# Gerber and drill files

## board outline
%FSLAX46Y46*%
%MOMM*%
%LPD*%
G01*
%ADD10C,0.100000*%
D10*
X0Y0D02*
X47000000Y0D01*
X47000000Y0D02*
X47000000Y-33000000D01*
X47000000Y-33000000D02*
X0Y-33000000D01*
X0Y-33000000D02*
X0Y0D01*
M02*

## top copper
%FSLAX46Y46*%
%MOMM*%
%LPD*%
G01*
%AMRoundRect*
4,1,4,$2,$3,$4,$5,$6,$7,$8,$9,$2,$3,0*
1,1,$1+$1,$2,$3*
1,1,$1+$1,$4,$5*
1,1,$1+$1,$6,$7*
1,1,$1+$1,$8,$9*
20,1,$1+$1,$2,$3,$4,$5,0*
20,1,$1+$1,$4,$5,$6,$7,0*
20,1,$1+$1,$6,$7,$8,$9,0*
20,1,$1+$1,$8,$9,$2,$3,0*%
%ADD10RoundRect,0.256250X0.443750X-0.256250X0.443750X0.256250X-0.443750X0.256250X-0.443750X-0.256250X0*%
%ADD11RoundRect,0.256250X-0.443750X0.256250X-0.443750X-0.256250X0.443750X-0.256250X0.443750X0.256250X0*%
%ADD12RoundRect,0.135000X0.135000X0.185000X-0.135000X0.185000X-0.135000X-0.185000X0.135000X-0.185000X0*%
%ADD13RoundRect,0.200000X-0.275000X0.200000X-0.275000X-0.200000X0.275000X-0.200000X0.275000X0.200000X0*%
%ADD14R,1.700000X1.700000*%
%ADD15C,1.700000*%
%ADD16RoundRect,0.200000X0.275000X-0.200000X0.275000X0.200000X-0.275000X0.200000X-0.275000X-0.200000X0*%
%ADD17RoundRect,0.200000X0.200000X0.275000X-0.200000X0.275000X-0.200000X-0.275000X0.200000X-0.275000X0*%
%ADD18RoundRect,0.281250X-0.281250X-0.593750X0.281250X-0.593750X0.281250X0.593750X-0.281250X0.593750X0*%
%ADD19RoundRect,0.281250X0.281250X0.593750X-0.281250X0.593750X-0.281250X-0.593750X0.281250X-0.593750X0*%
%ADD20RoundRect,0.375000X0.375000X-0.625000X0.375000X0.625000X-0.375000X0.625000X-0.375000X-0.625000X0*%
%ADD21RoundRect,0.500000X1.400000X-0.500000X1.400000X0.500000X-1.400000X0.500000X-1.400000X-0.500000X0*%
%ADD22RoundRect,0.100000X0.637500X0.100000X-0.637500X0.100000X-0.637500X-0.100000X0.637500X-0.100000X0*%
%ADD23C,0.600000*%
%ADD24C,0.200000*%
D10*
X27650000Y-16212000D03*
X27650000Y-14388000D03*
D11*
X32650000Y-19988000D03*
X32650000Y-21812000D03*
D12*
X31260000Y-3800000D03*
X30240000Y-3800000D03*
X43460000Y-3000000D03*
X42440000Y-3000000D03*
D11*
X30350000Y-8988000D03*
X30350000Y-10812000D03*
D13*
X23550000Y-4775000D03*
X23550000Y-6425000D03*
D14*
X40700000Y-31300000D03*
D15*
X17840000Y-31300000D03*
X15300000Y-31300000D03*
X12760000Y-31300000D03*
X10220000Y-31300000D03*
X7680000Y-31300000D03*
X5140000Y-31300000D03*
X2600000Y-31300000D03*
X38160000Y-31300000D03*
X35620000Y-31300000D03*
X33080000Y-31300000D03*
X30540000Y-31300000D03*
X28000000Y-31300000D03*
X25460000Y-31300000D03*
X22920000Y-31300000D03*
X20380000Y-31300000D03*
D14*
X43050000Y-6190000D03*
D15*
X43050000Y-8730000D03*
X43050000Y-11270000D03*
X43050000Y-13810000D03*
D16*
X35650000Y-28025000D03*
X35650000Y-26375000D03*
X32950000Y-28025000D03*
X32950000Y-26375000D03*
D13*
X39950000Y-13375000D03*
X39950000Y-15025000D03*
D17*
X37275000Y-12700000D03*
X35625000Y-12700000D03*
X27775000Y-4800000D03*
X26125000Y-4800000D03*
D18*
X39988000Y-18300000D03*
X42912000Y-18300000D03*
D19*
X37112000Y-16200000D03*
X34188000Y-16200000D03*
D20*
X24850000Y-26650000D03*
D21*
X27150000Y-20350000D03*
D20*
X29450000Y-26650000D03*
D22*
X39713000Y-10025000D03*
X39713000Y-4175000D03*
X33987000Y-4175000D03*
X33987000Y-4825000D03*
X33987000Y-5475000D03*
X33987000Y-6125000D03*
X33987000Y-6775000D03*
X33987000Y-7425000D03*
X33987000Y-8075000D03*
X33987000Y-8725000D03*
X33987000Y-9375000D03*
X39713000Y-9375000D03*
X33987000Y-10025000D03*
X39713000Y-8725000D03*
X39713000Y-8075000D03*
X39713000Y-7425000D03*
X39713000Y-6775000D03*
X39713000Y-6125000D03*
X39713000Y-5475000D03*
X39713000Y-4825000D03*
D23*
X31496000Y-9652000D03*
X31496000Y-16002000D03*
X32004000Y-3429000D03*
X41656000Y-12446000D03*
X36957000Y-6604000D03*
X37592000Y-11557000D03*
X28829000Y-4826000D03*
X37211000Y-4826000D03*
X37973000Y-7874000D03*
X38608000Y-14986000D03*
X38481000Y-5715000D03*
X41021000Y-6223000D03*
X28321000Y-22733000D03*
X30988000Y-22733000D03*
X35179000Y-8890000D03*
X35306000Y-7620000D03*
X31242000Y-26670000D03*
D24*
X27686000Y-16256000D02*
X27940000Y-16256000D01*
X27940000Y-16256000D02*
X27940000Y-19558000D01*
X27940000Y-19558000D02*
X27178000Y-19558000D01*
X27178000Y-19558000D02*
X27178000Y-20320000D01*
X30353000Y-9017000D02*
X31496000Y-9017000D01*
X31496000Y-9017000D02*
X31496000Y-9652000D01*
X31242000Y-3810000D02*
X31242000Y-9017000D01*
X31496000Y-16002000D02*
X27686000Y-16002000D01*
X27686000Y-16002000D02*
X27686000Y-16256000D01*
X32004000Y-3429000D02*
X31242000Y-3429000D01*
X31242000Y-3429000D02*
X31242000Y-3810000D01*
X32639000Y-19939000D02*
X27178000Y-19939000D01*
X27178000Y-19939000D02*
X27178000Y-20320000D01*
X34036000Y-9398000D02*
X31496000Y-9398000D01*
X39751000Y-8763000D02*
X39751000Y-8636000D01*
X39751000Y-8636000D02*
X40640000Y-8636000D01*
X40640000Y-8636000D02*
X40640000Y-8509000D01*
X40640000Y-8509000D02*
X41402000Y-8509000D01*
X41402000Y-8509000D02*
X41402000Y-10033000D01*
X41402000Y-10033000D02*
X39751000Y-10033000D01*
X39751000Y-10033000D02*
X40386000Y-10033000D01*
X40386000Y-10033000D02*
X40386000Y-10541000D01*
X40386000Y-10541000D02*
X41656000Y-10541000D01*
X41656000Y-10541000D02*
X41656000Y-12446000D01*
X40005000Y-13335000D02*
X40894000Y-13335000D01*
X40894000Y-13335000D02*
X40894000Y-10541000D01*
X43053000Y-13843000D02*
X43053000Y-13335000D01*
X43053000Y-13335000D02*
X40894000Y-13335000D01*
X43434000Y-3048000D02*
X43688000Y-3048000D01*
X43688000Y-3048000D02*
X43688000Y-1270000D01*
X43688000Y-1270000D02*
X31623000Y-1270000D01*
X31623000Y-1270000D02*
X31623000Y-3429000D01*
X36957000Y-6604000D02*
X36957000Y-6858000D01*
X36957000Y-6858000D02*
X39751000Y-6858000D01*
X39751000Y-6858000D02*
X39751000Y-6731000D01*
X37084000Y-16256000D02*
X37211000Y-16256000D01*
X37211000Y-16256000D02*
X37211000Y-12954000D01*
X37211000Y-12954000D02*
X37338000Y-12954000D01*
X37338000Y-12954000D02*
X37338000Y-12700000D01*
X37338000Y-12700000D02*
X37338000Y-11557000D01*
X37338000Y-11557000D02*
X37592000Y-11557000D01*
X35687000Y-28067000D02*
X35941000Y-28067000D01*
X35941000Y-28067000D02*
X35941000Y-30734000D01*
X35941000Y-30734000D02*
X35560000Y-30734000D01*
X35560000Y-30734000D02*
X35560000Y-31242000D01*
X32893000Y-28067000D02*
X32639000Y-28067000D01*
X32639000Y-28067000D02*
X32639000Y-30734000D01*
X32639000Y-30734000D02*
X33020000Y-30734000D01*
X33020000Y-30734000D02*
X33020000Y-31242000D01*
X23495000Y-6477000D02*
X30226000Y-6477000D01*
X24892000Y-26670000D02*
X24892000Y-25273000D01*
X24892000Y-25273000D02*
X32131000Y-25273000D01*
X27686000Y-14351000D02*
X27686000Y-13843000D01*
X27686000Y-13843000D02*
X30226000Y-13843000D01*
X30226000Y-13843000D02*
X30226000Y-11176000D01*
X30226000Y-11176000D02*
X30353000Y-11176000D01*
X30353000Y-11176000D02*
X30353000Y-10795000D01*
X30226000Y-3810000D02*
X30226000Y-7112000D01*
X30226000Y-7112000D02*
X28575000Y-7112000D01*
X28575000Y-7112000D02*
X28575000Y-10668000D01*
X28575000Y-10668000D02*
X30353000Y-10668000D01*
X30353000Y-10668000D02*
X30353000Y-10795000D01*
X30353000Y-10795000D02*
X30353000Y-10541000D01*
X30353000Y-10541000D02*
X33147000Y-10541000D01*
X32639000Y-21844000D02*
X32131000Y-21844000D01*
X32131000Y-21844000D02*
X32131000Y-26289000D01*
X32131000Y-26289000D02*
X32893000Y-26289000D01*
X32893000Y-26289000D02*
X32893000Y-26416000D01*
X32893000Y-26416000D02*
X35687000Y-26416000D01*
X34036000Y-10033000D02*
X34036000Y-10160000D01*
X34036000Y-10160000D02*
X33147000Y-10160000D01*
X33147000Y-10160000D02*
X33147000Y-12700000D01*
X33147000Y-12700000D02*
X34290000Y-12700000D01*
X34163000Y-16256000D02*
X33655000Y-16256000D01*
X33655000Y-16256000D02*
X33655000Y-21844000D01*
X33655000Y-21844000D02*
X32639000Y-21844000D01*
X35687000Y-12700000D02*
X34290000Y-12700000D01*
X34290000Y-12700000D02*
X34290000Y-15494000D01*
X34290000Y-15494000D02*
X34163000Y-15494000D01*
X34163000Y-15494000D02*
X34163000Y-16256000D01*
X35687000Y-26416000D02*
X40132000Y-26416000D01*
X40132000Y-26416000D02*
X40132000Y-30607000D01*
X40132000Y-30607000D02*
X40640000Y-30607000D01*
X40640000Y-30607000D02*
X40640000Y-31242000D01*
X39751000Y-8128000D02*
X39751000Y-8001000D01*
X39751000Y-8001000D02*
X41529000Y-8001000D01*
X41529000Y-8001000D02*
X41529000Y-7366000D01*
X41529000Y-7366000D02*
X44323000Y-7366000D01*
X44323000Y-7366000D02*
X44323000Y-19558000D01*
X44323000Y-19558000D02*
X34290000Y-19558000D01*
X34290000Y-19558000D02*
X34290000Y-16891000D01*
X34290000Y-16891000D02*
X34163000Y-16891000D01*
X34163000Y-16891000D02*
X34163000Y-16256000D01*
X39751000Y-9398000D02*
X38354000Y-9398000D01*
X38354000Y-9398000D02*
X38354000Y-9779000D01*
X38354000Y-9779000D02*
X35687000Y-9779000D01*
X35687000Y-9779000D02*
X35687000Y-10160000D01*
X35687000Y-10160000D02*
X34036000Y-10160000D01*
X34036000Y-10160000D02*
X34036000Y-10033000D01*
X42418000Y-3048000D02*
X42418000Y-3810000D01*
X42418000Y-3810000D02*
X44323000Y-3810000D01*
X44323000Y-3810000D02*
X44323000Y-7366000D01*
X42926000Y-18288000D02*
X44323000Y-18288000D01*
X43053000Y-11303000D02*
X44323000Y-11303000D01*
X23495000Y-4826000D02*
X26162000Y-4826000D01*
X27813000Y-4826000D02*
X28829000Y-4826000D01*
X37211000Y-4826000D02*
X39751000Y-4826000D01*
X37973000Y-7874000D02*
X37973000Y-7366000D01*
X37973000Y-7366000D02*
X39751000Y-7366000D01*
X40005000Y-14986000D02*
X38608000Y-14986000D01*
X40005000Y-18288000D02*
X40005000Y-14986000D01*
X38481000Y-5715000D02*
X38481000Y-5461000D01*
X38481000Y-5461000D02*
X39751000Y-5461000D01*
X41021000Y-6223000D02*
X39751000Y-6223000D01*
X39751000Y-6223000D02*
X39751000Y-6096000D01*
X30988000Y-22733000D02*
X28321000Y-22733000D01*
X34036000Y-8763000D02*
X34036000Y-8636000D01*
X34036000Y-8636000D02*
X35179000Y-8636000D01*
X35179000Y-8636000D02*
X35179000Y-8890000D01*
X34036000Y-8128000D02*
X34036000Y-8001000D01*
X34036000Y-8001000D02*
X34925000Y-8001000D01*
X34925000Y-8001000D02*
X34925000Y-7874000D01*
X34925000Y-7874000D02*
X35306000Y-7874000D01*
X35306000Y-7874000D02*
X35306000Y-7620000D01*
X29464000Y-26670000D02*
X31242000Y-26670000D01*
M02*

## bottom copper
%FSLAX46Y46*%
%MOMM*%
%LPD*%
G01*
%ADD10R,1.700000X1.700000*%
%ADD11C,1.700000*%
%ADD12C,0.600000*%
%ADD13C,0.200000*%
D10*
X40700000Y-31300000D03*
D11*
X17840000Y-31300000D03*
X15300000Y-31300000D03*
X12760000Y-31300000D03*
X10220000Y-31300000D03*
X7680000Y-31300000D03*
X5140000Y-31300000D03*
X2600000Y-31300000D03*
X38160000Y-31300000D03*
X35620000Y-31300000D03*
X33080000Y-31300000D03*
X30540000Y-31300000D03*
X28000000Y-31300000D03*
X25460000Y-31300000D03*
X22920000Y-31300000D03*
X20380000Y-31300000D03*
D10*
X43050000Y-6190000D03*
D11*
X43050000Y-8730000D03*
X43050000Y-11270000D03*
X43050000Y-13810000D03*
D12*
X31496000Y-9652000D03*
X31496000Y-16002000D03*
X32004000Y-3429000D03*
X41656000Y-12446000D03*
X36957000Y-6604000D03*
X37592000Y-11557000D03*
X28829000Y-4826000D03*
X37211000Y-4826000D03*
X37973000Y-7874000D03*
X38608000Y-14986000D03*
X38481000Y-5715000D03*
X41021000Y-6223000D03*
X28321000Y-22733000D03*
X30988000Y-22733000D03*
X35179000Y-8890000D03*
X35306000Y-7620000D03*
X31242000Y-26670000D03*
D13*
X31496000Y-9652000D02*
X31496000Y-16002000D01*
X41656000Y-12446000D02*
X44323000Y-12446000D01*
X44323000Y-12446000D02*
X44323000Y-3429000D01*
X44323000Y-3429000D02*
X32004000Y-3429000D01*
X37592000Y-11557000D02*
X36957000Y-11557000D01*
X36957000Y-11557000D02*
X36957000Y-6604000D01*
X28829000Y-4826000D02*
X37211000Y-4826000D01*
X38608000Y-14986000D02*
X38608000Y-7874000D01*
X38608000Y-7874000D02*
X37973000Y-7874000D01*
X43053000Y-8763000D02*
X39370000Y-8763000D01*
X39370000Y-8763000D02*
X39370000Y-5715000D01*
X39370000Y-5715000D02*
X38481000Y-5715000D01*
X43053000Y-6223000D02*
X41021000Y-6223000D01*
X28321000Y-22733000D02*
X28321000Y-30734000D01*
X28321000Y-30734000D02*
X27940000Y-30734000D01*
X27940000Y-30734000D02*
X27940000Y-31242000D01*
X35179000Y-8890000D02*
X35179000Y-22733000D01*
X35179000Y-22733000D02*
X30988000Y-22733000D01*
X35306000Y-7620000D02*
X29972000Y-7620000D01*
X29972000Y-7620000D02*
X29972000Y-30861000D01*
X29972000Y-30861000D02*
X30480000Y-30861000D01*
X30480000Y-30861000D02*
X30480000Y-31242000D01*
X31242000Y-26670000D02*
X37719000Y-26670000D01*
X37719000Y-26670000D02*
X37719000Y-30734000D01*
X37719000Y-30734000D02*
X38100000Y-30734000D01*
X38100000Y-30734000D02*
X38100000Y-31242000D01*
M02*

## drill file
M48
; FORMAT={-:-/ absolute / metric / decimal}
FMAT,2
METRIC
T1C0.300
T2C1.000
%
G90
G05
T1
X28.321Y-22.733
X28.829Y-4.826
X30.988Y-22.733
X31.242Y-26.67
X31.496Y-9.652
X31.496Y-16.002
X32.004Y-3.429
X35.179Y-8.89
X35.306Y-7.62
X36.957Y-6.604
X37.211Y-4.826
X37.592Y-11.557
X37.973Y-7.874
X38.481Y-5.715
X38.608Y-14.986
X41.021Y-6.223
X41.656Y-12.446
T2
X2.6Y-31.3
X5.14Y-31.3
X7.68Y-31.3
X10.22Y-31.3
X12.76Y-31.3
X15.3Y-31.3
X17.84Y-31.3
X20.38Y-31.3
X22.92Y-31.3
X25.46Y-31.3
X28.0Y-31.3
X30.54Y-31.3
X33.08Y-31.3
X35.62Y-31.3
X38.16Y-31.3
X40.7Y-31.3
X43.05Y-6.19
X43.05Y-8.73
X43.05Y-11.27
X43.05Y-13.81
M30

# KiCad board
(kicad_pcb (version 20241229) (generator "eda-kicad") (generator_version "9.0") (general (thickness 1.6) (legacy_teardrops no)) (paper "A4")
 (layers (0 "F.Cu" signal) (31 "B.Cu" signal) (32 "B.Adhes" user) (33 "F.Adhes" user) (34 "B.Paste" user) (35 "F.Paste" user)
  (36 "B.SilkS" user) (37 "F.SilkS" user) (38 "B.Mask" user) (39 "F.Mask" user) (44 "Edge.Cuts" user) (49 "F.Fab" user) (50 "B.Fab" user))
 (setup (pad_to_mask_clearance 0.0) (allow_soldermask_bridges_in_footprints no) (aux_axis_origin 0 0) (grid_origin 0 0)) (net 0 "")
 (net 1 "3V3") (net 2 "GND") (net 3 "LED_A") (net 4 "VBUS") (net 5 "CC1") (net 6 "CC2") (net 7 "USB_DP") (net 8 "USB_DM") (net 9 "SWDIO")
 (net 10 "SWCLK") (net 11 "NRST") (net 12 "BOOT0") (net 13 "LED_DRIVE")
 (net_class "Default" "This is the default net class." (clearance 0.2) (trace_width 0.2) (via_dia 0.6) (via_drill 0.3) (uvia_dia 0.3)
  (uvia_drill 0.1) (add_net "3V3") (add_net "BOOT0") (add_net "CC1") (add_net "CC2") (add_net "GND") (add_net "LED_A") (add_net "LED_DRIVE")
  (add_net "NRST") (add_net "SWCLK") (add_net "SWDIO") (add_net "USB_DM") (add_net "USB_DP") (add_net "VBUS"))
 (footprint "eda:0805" (layer "F.Cu") (at 27.65 15.3 -270)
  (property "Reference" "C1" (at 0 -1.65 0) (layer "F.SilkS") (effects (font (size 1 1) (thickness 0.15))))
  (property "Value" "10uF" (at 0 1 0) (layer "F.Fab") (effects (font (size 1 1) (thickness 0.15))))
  (pad "1" smd roundrect (at -0.912 0 -270) (size 1.025 1.4) (roundrect_rratio 0.25) (layers "F.Cu" "F.Paste" "F.Mask") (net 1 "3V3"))
  (pad "2" smd roundrect (at 0.912 0 -270) (size 1.025 1.4) (roundrect_rratio 0.25) (layers "F.Cu" "F.Paste" "F.Mask") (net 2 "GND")))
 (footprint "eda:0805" (layer "F.Cu") (at 32.65 20.9 -90)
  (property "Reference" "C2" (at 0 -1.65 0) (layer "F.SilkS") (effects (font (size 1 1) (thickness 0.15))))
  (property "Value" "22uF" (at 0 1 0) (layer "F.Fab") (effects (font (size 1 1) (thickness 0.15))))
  (pad "1" smd roundrect (at -0.912 0 -90) (size 1.025 1.4) (roundrect_rratio 0.25) (layers "F.Cu" "F.Paste" "F.Mask") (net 1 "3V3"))
  (pad "2" smd roundrect (at 0.912 0 -90) (size 1.025 1.4) (roundrect_rratio 0.25) (layers "F.Cu" "F.Paste" "F.Mask") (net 2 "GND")))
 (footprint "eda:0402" (layer "F.Cu") (at 30.75 3.8 -180)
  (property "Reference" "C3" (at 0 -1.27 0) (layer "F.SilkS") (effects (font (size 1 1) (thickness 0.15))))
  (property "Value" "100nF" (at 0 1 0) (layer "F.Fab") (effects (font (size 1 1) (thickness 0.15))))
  (pad "1" smd roundrect (at -0.51 0 -180) (size 0.54 0.64) (roundrect_rratio 0.25) (layers "F.Cu" "F.Paste" "F.Mask") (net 1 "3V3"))
  (pad "2" smd roundrect (at 0.51 0 -180) (size 0.54 0.64) (roundrect_rratio 0.25) (layers "F.Cu" "F.Paste" "F.Mask") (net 2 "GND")))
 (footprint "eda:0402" (layer "F.Cu") (at 42.95 3 -180)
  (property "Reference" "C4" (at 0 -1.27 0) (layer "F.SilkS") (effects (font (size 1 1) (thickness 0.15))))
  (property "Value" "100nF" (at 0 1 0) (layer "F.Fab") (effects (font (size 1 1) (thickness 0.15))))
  (pad "1" smd roundrect (at -0.51 0 -180) (size 0.54 0.64) (roundrect_rratio 0.25) (layers "F.Cu" "F.Paste" "F.Mask") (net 1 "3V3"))
  (pad "2" smd roundrect (at 0.51 0 -180) (size 0.54 0.64) (roundrect_rratio 0.25) (layers "F.Cu" "F.Paste" "F.Mask") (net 2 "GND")))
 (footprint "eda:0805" (layer "F.Cu") (at 30.35 9.9 -90)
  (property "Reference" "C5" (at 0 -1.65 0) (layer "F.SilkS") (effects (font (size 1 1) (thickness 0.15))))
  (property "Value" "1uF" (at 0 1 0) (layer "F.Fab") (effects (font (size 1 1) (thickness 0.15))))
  (pad "1" smd roundrect (at -0.912 0 -90) (size 1.025 1.4) (roundrect_rratio 0.25) (layers "F.Cu" "F.Paste" "F.Mask") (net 1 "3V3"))
  (pad "2" smd roundrect (at 0.912 0 -90) (size 1.025 1.4) (roundrect_rratio 0.25) (layers "F.Cu" "F.Paste" "F.Mask") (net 2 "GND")))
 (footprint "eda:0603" (layer "F.Cu") (at 23.55 5.6 -90)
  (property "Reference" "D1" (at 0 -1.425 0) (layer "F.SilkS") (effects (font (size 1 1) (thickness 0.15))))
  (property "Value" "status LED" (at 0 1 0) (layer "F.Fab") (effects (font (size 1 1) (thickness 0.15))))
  (pad "1" smd roundrect (at -0.825 0 -90) (size 0.8 0.95) (roundrect_rratio 0.25) (layers "F.Cu" "F.Paste" "F.Mask") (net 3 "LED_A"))
  (pad "2" smd roundrect (at 0.825 0 -90) (size 0.8 0.95) (roundrect_rratio 0.25) (layers "F.Cu" "F.Paste" "F.Mask") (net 2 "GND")))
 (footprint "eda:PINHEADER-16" (layer "F.Cu") (at 21.65 31.3 -180)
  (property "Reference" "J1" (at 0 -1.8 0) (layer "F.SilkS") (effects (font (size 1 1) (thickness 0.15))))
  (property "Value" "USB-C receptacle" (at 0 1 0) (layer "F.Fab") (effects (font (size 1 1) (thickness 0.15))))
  (pad "1" thru_hole rect (at -19.05 0 -180) (size 1.7 1.7) (drill 1) (layers "*.Cu" "*.Mask") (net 2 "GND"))
  (pad "10" thru_hole circle (at 3.81 0 -180) (size 1.7 1.7) (drill 1) (layers "*.Cu" "*.Mask"))
  (pad "11" thru_hole circle (at 6.35 0 -180) (size 1.7 1.7) (drill 1) (layers "*.Cu" "*.Mask"))
  (pad "12" thru_hole circle (at 8.89 0 -180) (size 1.7 1.7) (drill 1) (layers "*.Cu" "*.Mask"))
  (pad "13" thru_hole circle (at 11.43 0 -180) (size 1.7 1.7) (drill 1) (layers "*.Cu" "*.Mask"))
  (pad "14" thru_hole circle (at 13.97 0 -180) (size 1.7 1.7) (drill 1) (layers "*.Cu" "*.Mask"))
  (pad "15" thru_hole circle (at 16.51 0 -180) (size 1.7 1.7) (drill 1) (layers "*.Cu" "*.Mask"))
  (pad "16" thru_hole circle (at 19.05 0 -180) (size 1.7 1.7) (drill 1) (layers "*.Cu" "*.Mask"))
  (pad "2" thru_hole circle (at -16.51 0 -180) (size 1.7 1.7) (drill 1) (layers "*.Cu" "*.Mask") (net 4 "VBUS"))
  (pad "3" thru_hole circle (at -13.97 0 -180) (size 1.7 1.7) (drill 1) (layers "*.Cu" "*.Mask") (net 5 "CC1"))
  (pad "4" thru_hole circle (at -11.43 0 -180) (size 1.7 1.7) (drill 1) (layers "*.Cu" "*.Mask") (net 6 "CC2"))
  (pad "5" thru_hole circle (at -8.89 0 -180) (size 1.7 1.7) (drill 1) (layers "*.Cu" "*.Mask") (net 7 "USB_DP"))
  (pad "6" thru_hole circle (at -6.35 0 -180) (size 1.7 1.7) (drill 1) (layers "*.Cu" "*.Mask") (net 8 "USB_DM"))
  (pad "7" thru_hole circle (at -3.81 0 -180) (size 1.7 1.7) (drill 1) (layers "*.Cu" "*.Mask"))
  (pad "8" thru_hole circle (at -1.27 0 -180) (size 1.7 1.7) (drill 1) (layers "*.Cu" "*.Mask"))
  (pad "9" thru_hole circle (at 1.27 0 -180) (size 1.7 1.7) (drill 1) (layers "*.Cu" "*.Mask")))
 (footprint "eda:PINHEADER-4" (layer "F.Cu") (at 43.05 10 -90)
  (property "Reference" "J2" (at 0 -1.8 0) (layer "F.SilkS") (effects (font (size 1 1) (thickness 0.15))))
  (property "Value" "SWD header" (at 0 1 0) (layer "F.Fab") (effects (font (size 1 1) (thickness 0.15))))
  (pad "1" thru_hole rect (at -3.81 0 -90) (size 1.7 1.7) (drill 1) (layers "*.Cu" "*.Mask") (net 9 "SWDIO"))
  (pad "2" thru_hole circle (at -1.27 0 -90) (size 1.7 1.7) (drill 1) (layers "*.Cu" "*.Mask") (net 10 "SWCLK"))
  (pad "3" thru_hole circle (at 1.27 0 -90) (size 1.7 1.7) (drill 1) (layers "*.Cu" "*.Mask") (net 2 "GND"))
  (pad "4" thru_hole circle (at 3.81 0 -90) (size 1.7 1.7) (drill 1) (layers "*.Cu" "*.Mask") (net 1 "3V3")))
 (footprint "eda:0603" (layer "F.Cu") (at 35.65 27.2 -270)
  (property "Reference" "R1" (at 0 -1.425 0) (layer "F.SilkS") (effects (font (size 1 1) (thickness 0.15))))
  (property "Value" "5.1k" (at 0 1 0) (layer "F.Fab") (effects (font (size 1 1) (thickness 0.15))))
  (pad "1" smd roundrect (at -0.825 0 -270) (size 0.8 0.95) (roundrect_rratio 0.25) (layers "F.Cu" "F.Paste" "F.Mask") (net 5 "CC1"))
  (pad "2" smd roundrect (at 0.825 0 -270) (size 0.8 0.95) (roundrect_rratio 0.25) (layers "F.Cu" "F.Paste" "F.Mask") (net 2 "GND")))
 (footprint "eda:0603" (layer "F.Cu") (at 32.95 27.2 -270)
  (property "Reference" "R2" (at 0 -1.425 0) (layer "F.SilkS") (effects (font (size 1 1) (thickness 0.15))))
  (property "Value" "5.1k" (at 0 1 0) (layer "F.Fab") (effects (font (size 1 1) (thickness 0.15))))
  (pad "1" smd roundrect (at -0.825 0 -270) (size 0.8 0.95) (roundrect_rratio 0.25) (layers "F.Cu" "F.Paste" "F.Mask") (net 6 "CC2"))
  (pad "2" smd roundrect (at 0.825 0 -270) (size 0.8 0.95) (roundrect_rratio 0.25) (layers "F.Cu" "F.Paste" "F.Mask") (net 2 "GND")))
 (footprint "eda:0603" (layer "F.Cu") (at 39.95 14.2 -90)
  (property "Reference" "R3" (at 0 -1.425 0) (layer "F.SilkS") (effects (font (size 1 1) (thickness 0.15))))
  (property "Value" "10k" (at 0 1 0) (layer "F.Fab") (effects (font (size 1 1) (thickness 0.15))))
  (pad "1" smd roundrect (at -0.825 0 -90) (size 0.8 0.95) (roundrect_rratio 0.25) (layers "F.Cu" "F.Paste" "F.Mask") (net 1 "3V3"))
  (pad "2" smd roundrect (at 0.825 0 -90) (size 0.8 0.95) (roundrect_rratio 0.25) (layers "F.Cu" "F.Paste" "F.Mask") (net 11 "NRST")))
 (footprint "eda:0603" (layer "F.Cu") (at 36.45 12.7 -180)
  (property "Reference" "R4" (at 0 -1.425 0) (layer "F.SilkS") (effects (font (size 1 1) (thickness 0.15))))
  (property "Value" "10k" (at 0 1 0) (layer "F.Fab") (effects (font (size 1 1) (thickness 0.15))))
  (pad "1" smd roundrect (at -0.825 0 -180) (size 0.8 0.95) (roundrect_rratio 0.25) (layers "F.Cu" "F.Paste" "F.Mask") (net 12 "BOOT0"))
  (pad "2" smd roundrect (at 0.825 0 -180) (size 0.8 0.95) (roundrect_rratio 0.25) (layers "F.Cu" "F.Paste" "F.Mask") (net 2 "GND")))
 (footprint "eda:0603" (layer "F.Cu") (at 26.95 4.8 -180)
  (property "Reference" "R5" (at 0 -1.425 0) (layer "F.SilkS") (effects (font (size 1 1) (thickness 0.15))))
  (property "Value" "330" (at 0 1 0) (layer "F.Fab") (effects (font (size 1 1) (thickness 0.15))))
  (pad "1" smd roundrect (at -0.825 0 -180) (size 0.8 0.95) (roundrect_rratio 0.25) (layers "F.Cu" "F.Paste" "F.Mask") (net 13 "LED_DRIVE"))
  (pad "2" smd roundrect (at 0.825 0 -180) (size 0.8 0.95) (roundrect_rratio 0.25) (layers "F.Cu" "F.Paste" "F.Mask") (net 3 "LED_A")))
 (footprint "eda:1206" (layer "F.Cu") (at 41.45 18.3 0)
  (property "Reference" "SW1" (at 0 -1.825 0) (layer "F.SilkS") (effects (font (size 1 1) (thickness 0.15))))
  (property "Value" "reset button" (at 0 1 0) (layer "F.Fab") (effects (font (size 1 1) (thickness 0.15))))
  (pad "1" smd roundrect (at -1.462 0 0) (size 1.125 1.75) (roundrect_rratio 0.25) (layers "F.Cu" "F.Paste" "F.Mask") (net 11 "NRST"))
  (pad "2" smd roundrect (at 1.462 0 0) (size 1.125 1.75) (roundrect_rratio 0.25) (layers "F.Cu" "F.Paste" "F.Mask") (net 2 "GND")))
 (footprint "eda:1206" (layer "F.Cu") (at 35.65 16.2 -180)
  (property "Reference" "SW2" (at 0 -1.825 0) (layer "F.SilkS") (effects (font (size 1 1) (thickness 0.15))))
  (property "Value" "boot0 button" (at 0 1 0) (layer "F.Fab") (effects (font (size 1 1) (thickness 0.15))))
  (pad "1" smd roundrect (at -1.462 0 -180) (size 1.125 1.75) (roundrect_rratio 0.25) (layers "F.Cu" "F.Paste" "F.Mask") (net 12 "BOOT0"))
  (pad "2" smd roundrect (at 1.462 0 -180) (size 1.125 1.75) (roundrect_rratio 0.25) (layers "F.Cu" "F.Paste" "F.Mask") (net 2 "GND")))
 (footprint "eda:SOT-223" (layer "F.Cu") (at 27.15 23.5 -270)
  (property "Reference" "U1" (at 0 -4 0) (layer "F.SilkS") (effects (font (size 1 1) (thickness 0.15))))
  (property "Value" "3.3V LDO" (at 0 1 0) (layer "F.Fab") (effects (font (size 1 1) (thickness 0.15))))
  (pad "1" smd roundrect (at -3.15 -2.3 -270) (size 2 1.5) (roundrect_rratio 0.25) (layers "F.Cu" "F.Paste" "F.Mask") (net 2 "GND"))
  (pad "2" smd roundrect (at 3.15 0 -270) (size 2 3.8) (roundrect_rratio 0.25) (layers "F.Cu" "F.Paste" "F.Mask") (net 1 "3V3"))
  (pad "3" smd roundrect (at -3.15 2.3 -270) (size 2 1.5) (roundrect_rratio 0.25) (layers "F.Cu" "F.Paste" "F.Mask") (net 4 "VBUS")))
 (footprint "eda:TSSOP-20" (layer "F.Cu") (at 36.85 7.1 -180)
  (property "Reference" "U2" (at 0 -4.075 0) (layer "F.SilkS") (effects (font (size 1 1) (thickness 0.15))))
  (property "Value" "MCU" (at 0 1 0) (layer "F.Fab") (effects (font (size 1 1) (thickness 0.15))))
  (pad "1" smd roundrect (at -2.863 -2.925 -180) (size 1.475 0.4) (roundrect_rratio 0.25) (layers "F.Cu" "F.Paste" "F.Mask") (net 1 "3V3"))
  (pad "10" smd roundrect (at -2.863 2.925 -180) (size 1.475 0.4) (roundrect_rratio 0.25) (layers "F.Cu" "F.Paste" "F.Mask"))
  (pad "11" smd roundrect (at 2.863 2.925 -180) (size 1.475 0.4) (roundrect_rratio 0.25) (layers "F.Cu" "F.Paste" "F.Mask"))
  (pad "12" smd roundrect (at 2.863 2.275 -180) (size 1.475 0.4) (roundrect_rratio 0.25) (layers "F.Cu" "F.Paste" "F.Mask"))
  (pad "13" smd roundrect (at 2.863 1.625 -180) (size 1.475 0.4) (roundrect_rratio 0.25) (layers "F.Cu" "F.Paste" "F.Mask"))
  (pad "14" smd roundrect (at 2.863 0.975 -180) (size 1.475 0.4) (roundrect_rratio 0.25) (layers "F.Cu" "F.Paste" "F.Mask"))
  (pad "15" smd roundrect (at 2.863 0.325 -180) (size 1.475 0.4) (roundrect_rratio 0.25) (layers "F.Cu" "F.Paste" "F.Mask"))
  (pad "16" smd roundrect (at 2.863 -0.325 -180) (size 1.475 0.4) (roundrect_rratio 0.25) (layers "F.Cu" "F.Paste" "F.Mask"))
  (pad "17" smd roundrect (at 2.863 -0.975 -180) (size 1.475 0.4) (roundrect_rratio 0.25) (layers "F.Cu" "F.Paste" "F.Mask")
   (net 7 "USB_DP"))
  (pad "18" smd roundrect (at 2.863 -1.625 -180) (size 1.475 0.4) (roundrect_rratio 0.25) (layers "F.Cu" "F.Paste" "F.Mask")
   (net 8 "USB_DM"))
  (pad "19" smd roundrect (at 2.863 -2.275 -180) (size 1.475 0.4) (roundrect_rratio 0.25) (layers "F.Cu" "F.Paste" "F.Mask") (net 1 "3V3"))
  (pad "2" smd roundrect (at -2.863 -2.275 -180) (size 1.475 0.4) (roundrect_rratio 0.25) (layers "F.Cu" "F.Paste" "F.Mask") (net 2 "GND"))
  (pad "20" smd roundrect (at 2.863 -2.925 -180) (size 1.475 0.4) (roundrect_rratio 0.25) (layers "F.Cu" "F.Paste" "F.Mask") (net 2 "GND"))
  (pad "3" smd roundrect (at -2.863 -1.625 -180) (size 1.475 0.4) (roundrect_rratio 0.25) (layers "F.Cu" "F.Paste" "F.Mask") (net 1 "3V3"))
  (pad "4" smd roundrect (at -2.863 -0.975 -180) (size 1.475 0.4) (roundrect_rratio 0.25) (layers "F.Cu" "F.Paste" "F.Mask") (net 2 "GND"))
  (pad "5" smd roundrect (at -2.863 -0.325 -180) (size 1.475 0.4) (roundrect_rratio 0.25) (layers "F.Cu" "F.Paste" "F.Mask") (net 11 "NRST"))
  (pad "6" smd roundrect (at -2.863 0.325 -180) (size 1.475 0.4) (roundrect_rratio 0.25) (layers "F.Cu" "F.Paste" "F.Mask") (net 12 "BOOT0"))
  (pad "7" smd roundrect (at -2.863 0.975 -180) (size 1.475 0.4) (roundrect_rratio 0.25) (layers "F.Cu" "F.Paste" "F.Mask") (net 9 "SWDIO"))
  (pad "8" smd roundrect (at -2.863 1.625 -180) (size 1.475 0.4) (roundrect_rratio 0.25) (layers "F.Cu" "F.Paste" "F.Mask") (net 10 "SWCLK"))
  (pad "9" smd roundrect (at -2.863 2.275 -180) (size 1.475 0.4) (roundrect_rratio 0.25) (layers "F.Cu" "F.Paste" "F.Mask")
   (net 13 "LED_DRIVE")))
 (segment (start 31.496 9.652) (end 31.496 16.002) (width 0.2) (layer "B.Cu") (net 1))
 (segment (start 41.656 12.446) (end 44.323 12.446) (width 0.2) (layer "B.Cu") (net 1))
 (segment (start 44.323 12.446) (end 44.323 3.429) (width 0.2) (layer "B.Cu") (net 1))
 (segment (start 44.323 3.429) (end 32.004 3.429) (width 0.2) (layer "B.Cu") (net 1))
 (segment (start 27.686 16.256) (end 27.94 16.256) (width 0.2) (layer "F.Cu") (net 1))
 (segment (start 27.94 16.256) (end 27.94 19.558) (width 0.2) (layer "F.Cu") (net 1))
 (segment (start 27.94 19.558) (end 27.178 19.558) (width 0.2) (layer "F.Cu") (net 1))
 (segment (start 27.178 19.558) (end 27.178 20.32) (width 0.2) (layer "F.Cu") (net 1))
 (segment (start 30.353 9.017) (end 31.496 9.017) (width 0.2) (layer "F.Cu") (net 1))
 (segment (start 31.496 9.017) (end 31.496 9.652) (width 0.2) (layer "F.Cu") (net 1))
 (segment (start 31.242 3.81) (end 31.242 9.017) (width 0.2) (layer "F.Cu") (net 1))
 (segment (start 31.496 16.002) (end 27.686 16.002) (width 0.2) (layer "F.Cu") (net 1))
 (segment (start 27.686 16.002) (end 27.686 16.256) (width 0.2) (layer "F.Cu") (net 1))
 (segment (start 32.004 3.429) (end 31.242 3.429) (width 0.2) (layer "F.Cu") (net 1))
 (segment (start 31.242 3.429) (end 31.242 3.81) (width 0.2) (layer "F.Cu") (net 1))
 (segment (start 32.639 19.939) (end 27.178 19.939) (width 0.2) (layer "F.Cu") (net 1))
 (segment (start 27.178 19.939) (end 27.178 20.32) (width 0.2) (layer "F.Cu") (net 1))
 (segment (start 34.036 9.398) (end 31.496 9.398) (width 0.2) (layer "F.Cu") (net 1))
 (segment (start 39.751 8.763) (end 39.751 8.636) (width 0.2) (layer "F.Cu") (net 1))
 (segment (start 39.751 8.636) (end 40.64 8.636) (width 0.2) (layer "F.Cu") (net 1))
 (segment (start 40.64 8.636) (end 40.64 8.509) (width 0.2) (layer "F.Cu") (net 1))
 (segment (start 40.64 8.509) (end 41.402 8.509) (width 0.2) (layer "F.Cu") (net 1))
 (segment (start 41.402 8.509) (end 41.402 10.033) (width 0.2) (layer "F.Cu") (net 1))
 (segment (start 41.402 10.033) (end 39.751 10.033) (width 0.2) (layer "F.Cu") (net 1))
 (segment (start 39.751 10.033) (end 40.386 10.033) (width 0.2) (layer "F.Cu") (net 1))
 (segment (start 40.386 10.033) (end 40.386 10.541) (width 0.2) (layer "F.Cu") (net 1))
 (segment (start 40.386 10.541) (end 41.656 10.541) (width 0.2) (layer "F.Cu") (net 1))
 (segment (start 41.656 10.541) (end 41.656 12.446) (width 0.2) (layer "F.Cu") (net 1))
 (segment (start 40.005 13.335) (end 40.894 13.335) (width 0.2) (layer "F.Cu") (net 1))
 (segment (start 40.894 13.335) (end 40.894 10.541) (width 0.2) (layer "F.Cu") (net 1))
 (segment (start 43.053 13.843) (end 43.053 13.335) (width 0.2) (layer "F.Cu") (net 1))
 (segment (start 43.053 13.335) (end 40.894 13.335) (width 0.2) (layer "F.Cu") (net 1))
 (segment (start 43.434 3.048) (end 43.688 3.048) (width 0.2) (layer "F.Cu") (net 1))
 (segment (start 43.688 3.048) (end 43.688 1.27) (width 0.2) (layer "F.Cu") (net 1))
 (segment (start 43.688 1.27) (end 31.623 1.27) (width 0.2) (layer "F.Cu") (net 1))
 (segment (start 31.623 1.27) (end 31.623 3.429) (width 0.2) (layer "F.Cu") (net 1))
 (segment (start 37.592 11.557) (end 36.957 11.557) (width 0.2) (layer "B.Cu") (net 12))
 (segment (start 36.957 11.557) (end 36.957 6.604) (width 0.2) (layer "B.Cu") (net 12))
 (segment (start 36.957 6.604) (end 36.957 6.858) (width 0.2) (layer "F.Cu") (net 12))
 (segment (start 36.957 6.858) (end 39.751 6.858) (width 0.2) (layer "F.Cu") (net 12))
 (segment (start 39.751 6.858) (end 39.751 6.731) (width 0.2) (layer "F.Cu") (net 12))
 (segment (start 37.084 16.256) (end 37.211 16.256) (width 0.2) (layer "F.Cu") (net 12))
 (segment (start 37.211 16.256) (end 37.211 12.954) (width 0.2) (layer "F.Cu") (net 12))
 (segment (start 37.211 12.954) (end 37.338 12.954) (width 0.2) (layer "F.Cu") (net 12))
 (segment (start 37.338 12.954) (end 37.338 12.7) (width 0.2) (layer "F.Cu") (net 12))
 (segment (start 37.338 12.7) (end 37.338 11.557) (width 0.2) (layer "F.Cu") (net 12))
 (segment (start 37.338 11.557) (end 37.592 11.557) (width 0.2) (layer "F.Cu") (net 12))
 (segment (start 35.687 28.067) (end 35.941 28.067) (width 0.2) (layer "F.Cu") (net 5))
 (segment (start 35.941 28.067) (end 35.941 30.734) (width 0.2) (layer "F.Cu") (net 5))
 (segment (start 35.941 30.734) (end 35.56 30.734) (width 0.2) (layer "F.Cu") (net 5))
 (segment (start 35.56 30.734) (end 35.56 31.242) (width 0.2) (layer "F.Cu") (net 5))
 (segment (start 32.893 28.067) (end 32.639 28.067) (width 0.2) (layer "F.Cu") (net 6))
 (segment (start 32.639 28.067) (end 32.639 30.734) (width 0.2) (layer "F.Cu") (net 6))
 (segment (start 32.639 30.734) (end 33.02 30.734) (width 0.2) (layer "F.Cu") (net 6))
 (segment (start 33.02 30.734) (end 33.02 31.242) (width 0.2) (layer "F.Cu") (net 6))
 (segment (start 23.495 6.477) (end 30.226 6.477) (width 0.2) (layer "F.Cu") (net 2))
 (segment (start 24.892 26.67) (end 24.892 25.273) (width 0.2) (layer "F.Cu") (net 2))
 (segment (start 24.892 25.273) (end 32.131 25.273) (width 0.2) (layer "F.Cu") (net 2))
 (segment (start 27.686 14.351) (end 27.686 13.843) (width 0.2) (layer "F.Cu") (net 2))
 (segment (start 27.686 13.843) (end 30.226 13.843) (width 0.2) (layer "F.Cu") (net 2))
 (segment (start 30.226 13.843) (end 30.226 11.176) (width 0.2) (layer "F.Cu") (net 2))
 (segment (start 30.226 11.176) (end 30.353 11.176) (width 0.2) (layer "F.Cu") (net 2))
 (segment (start 30.353 11.176) (end 30.353 10.795) (width 0.2) (layer "F.Cu") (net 2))
 (segment (start 30.226 3.81) (end 30.226 7.112) (width 0.2) (layer "F.Cu") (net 2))
 (segment (start 30.226 7.112) (end 28.575 7.112) (width 0.2) (layer "F.Cu") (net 2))
 (segment (start 28.575 7.112) (end 28.575 10.668) (width 0.2) (layer "F.Cu") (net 2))
 (segment (start 28.575 10.668) (end 30.353 10.668) (width 0.2) (layer "F.Cu") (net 2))
 (segment (start 30.353 10.668) (end 30.353 10.795) (width 0.2) (layer "F.Cu") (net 2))
 (segment (start 30.353 10.795) (end 30.353 10.541) (width 0.2) (layer "F.Cu") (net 2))
 (segment (start 30.353 10.541) (end 33.147 10.541) (width 0.2) (layer "F.Cu") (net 2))
 (segment (start 32.639 21.844) (end 32.131 21.844) (width 0.2) (layer "F.Cu") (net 2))
 (segment (start 32.131 21.844) (end 32.131 26.289) (width 0.2) (layer "F.Cu") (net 2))
 (segment (start 32.131 26.289) (end 32.893 26.289) (width 0.2) (layer "F.Cu") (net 2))
 (segment (start 32.893 26.289) (end 32.893 26.416) (width 0.2) (layer "F.Cu") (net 2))
 (segment (start 32.893 26.416) (end 35.687 26.416) (width 0.2) (layer "F.Cu") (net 2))
 (segment (start 34.036 10.033) (end 34.036 10.16) (width 0.2) (layer "F.Cu") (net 2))
 (segment (start 34.036 10.16) (end 33.147 10.16) (width 0.2) (layer "F.Cu") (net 2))
 (segment (start 33.147 10.16) (end 33.147 12.7) (width 0.2) (layer "F.Cu") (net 2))
 (segment (start 33.147 12.7) (end 34.29 12.7) (width 0.2) (layer "F.Cu") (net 2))
 (segment (start 34.163 16.256) (end 33.655 16.256) (width 0.2) (layer "F.Cu") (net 2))
 (segment (start 33.655 16.256) (end 33.655 21.844) (width 0.2) (layer "F.Cu") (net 2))
 (segment (start 33.655 21.844) (end 32.639 21.844) (width 0.2) (layer "F.Cu") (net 2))
 (segment (start 35.687 12.7) (end 34.29 12.7) (width 0.2) (layer "F.Cu") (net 2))
 (segment (start 34.29 12.7) (end 34.29 15.494) (width 0.2) (layer "F.Cu") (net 2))
 (segment (start 34.29 15.494) (end 34.163 15.494) (width 0.2) (layer "F.Cu") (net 2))
 (segment (start 34.163 15.494) (end 34.163 16.256) (width 0.2) (layer "F.Cu") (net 2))
 (segment (start 35.687 26.416) (end 40.132 26.416) (width 0.2) (layer "F.Cu") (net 2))
 (segment (start 40.132 26.416) (end 40.132 30.607) (width 0.2) (layer "F.Cu") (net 2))
 (segment (start 40.132 30.607) (end 40.64 30.607) (width 0.2) (layer "F.Cu") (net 2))
 (segment (start 40.64 30.607) (end 40.64 31.242) (width 0.2) (layer "F.Cu") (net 2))
 (segment (start 39.751 8.128) (end 39.751 8.001) (width 0.2) (layer "F.Cu") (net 2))
 (segment (start 39.751 8.001) (end 41.529 8.001) (width 0.2) (layer "F.Cu") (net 2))
 (segment (start 41.529 8.001) (end 41.529 7.366) (width 0.2) (layer "F.Cu") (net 2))
 (segment (start 41.529 7.366) (end 44.323 7.366) (width 0.2) (layer "F.Cu") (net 2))
 (segment (start 44.323 7.366) (end 44.323 19.558) (width 0.2) (layer "F.Cu") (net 2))
 (segment (start 44.323 19.558) (end 34.29 19.558) (width 0.2) (layer "F.Cu") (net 2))
 (segment (start 34.29 19.558) (end 34.29 16.891) (width 0.2) (layer "F.Cu") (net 2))
 (segment (start 34.29 16.891) (end 34.163 16.891) (width 0.2) (layer "F.Cu") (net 2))
 (segment (start 34.163 16.891) (end 34.163 16.256) (width 0.2) (layer "F.Cu") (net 2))
 (segment (start 39.751 9.398) (end 38.354 9.398) (width 0.2) (layer "F.Cu") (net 2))
 (segment (start 38.354 9.398) (end 38.354 9.779) (width 0.2) (layer "F.Cu") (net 2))
 (segment (start 38.354 9.779) (end 35.687 9.779) (width 0.2) (layer "F.Cu") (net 2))
 (segment (start 35.687 9.779) (end 35.687 10.16) (width 0.2) (layer "F.Cu") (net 2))
 (segment (start 35.687 10.16) (end 34.036 10.16) (width 0.2) (layer "F.Cu") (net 2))
 (segment (start 34.036 10.16) (end 34.036 10.033) (width 0.2) (layer "F.Cu") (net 2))
 (segment (start 42.418 3.048) (end 42.418 3.81) (width 0.2) (layer "F.Cu") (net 2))
 (segment (start 42.418 3.81) (end 44.323 3.81) (width 0.2) (layer "F.Cu") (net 2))
 (segment (start 44.323 3.81) (end 44.323 7.366) (width 0.2) (layer "F.Cu") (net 2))
 (segment (start 42.926 18.288) (end 44.323 18.288) (width 0.2) (layer "F.Cu") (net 2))
 (segment (start 43.053 11.303) (end 44.323 11.303) (width 0.2) (layer "F.Cu") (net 2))
 (segment (start 23.495 4.826) (end 26.162 4.826) (width 0.2) (layer "F.Cu") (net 3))
 (segment (start 28.829 4.826) (end 37.211 4.826) (width 0.2) (layer "B.Cu") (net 13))
 (segment (start 27.813 4.826) (end 28.829 4.826) (width 0.2) (layer "F.Cu") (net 13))
 (segment (start 37.211 4.826) (end 39.751 4.826) (width 0.2) (layer "F.Cu") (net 13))
 (segment (start 38.608 14.986) (end 38.608 7.874) (width 0.2) (layer "B.Cu") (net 11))
 (segment (start 38.608 7.874) (end 37.973 7.874) (width 0.2) (layer "B.Cu") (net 11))
 (segment (start 37.973 7.874) (end 37.973 7.366) (width 0.2) (layer "F.Cu") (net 11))
 (segment (start 37.973 7.366) (end 39.751 7.366) (width 0.2) (layer "F.Cu") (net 11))
 (segment (start 40.005 14.986) (end 38.608 14.986) (width 0.2) (layer "F.Cu") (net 11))
 (segment (start 40.005 18.288) (end 40.005 14.986) (width 0.2) (layer "F.Cu") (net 11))
 (segment (start 43.053 8.763) (end 39.37 8.763) (width 0.2) (layer "B.Cu") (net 10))
 (segment (start 39.37 8.763) (end 39.37 5.715) (width 0.2) (layer "B.Cu") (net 10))
 (segment (start 39.37 5.715) (end 38.481 5.715) (width 0.2) (layer "B.Cu") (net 10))
 (segment (start 38.481 5.715) (end 38.481 5.461) (width 0.2) (layer "F.Cu") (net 10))
 (segment (start 38.481 5.461) (end 39.751 5.461) (width 0.2) (layer "F.Cu") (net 10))
 (segment (start 43.053 6.223) (end 41.021 6.223) (width 0.2) (layer "B.Cu") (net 9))
 (segment (start 41.021 6.223) (end 39.751 6.223) (width 0.2) (layer "F.Cu") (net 9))
 (segment (start 39.751 6.223) (end 39.751 6.096) (width 0.2) (layer "F.Cu") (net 9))
 (segment (start 28.321 22.733) (end 28.321 30.734) (width 0.2) (layer "B.Cu") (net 8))
 (segment (start 28.321 30.734) (end 27.94 30.734) (width 0.2) (layer "B.Cu") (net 8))
 (segment (start 27.94 30.734) (end 27.94 31.242) (width 0.2) (layer "B.Cu") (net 8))
 (segment (start 35.179 8.89) (end 35.179 22.733) (width 0.2) (layer "B.Cu") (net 8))
 (segment (start 35.179 22.733) (end 30.988 22.733) (width 0.2) (layer "B.Cu") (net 8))
 (segment (start 30.988 22.733) (end 28.321 22.733) (width 0.2) (layer "F.Cu") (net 8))
 (segment (start 34.036 8.763) (end 34.036 8.636) (width 0.2) (layer "F.Cu") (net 8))
 (segment (start 34.036 8.636) (end 35.179 8.636) (width 0.2) (layer "F.Cu") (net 8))
 (segment (start 35.179 8.636) (end 35.179 8.89) (width 0.2) (layer "F.Cu") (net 8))
 (segment (start 35.306 7.62) (end 29.972 7.62) (width 0.2) (layer "B.Cu") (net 7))
 (segment (start 29.972 7.62) (end 29.972 30.861) (width 0.2) (layer "B.Cu") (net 7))
 (segment (start 29.972 30.861) (end 30.48 30.861) (width 0.2) (layer "B.Cu") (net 7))
 (segment (start 30.48 30.861) (end 30.48 31.242) (width 0.2) (layer "B.Cu") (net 7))
 (segment (start 34.036 8.128) (end 34.036 8.001) (width 0.2) (layer "F.Cu") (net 7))
 (segment (start 34.036 8.001) (end 34.925 8.001) (width 0.2) (layer "F.Cu") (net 7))
 (segment (start 34.925 8.001) (end 34.925 7.874) (width 0.2) (layer "F.Cu") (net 7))
 (segment (start 34.925 7.874) (end 35.306 7.874) (width 0.2) (layer "F.Cu") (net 7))
 (segment (start 35.306 7.874) (end 35.306 7.62) (width 0.2) (layer "F.Cu") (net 7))
 (segment (start 31.242 26.67) (end 37.719 26.67) (width 0.2) (layer "B.Cu") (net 4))
 (segment (start 37.719 26.67) (end 37.719 30.734) (width 0.2) (layer "B.Cu") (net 4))
 (segment (start 37.719 30.734) (end 38.1 30.734) (width 0.2) (layer "B.Cu") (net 4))
 (segment (start 38.1 30.734) (end 38.1 31.242) (width 0.2) (layer "B.Cu") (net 4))
 (segment (start 29.464 26.67) (end 31.242 26.67) (width 0.2) (layer "F.Cu") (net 4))
 (via (at 31.496 9.652) (size 0.6) (drill 0.3) (layers "F.Cu" "B.Cu") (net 1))
 (via (at 31.496 16.002) (size 0.6) (drill 0.3) (layers "B.Cu" "F.Cu") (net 1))
 (via (at 32.004 3.429) (size 0.6) (drill 0.3) (layers "B.Cu" "F.Cu") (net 1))
 (via (at 41.656 12.446) (size 0.6) (drill 0.3) (layers "F.Cu" "B.Cu") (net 1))
 (via (at 36.957 6.604) (size 0.6) (drill 0.3) (layers "B.Cu" "F.Cu") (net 12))
 (via (at 37.592 11.557) (size 0.6) (drill 0.3) (layers "F.Cu" "B.Cu") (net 12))
 (via (at 28.829 4.826) (size 0.6) (drill 0.3) (layers "F.Cu" "B.Cu") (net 13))
 (via (at 37.211 4.826) (size 0.6) (drill 0.3) (layers "B.Cu" "F.Cu") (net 13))
 (via (at 37.973 7.874) (size 0.6) (drill 0.3) (layers "B.Cu" "F.Cu") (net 11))
 (via (at 38.608 14.986) (size 0.6) (drill 0.3) (layers "F.Cu" "B.Cu") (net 11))
 (via (at 38.481 5.715) (size 0.6) (drill 0.3) (layers "B.Cu" "F.Cu") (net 10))
 (via (at 41.021 6.223) (size 0.6) (drill 0.3) (layers "B.Cu" "F.Cu") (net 9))
 (via (at 28.321 22.733) (size 0.6) (drill 0.3) (layers "F.Cu" "B.Cu") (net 8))
 (via (at 30.988 22.733) (size 0.6) (drill 0.3) (layers "B.Cu" "F.Cu") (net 8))
 (via (at 35.179 8.89) (size 0.6) (drill 0.3) (layers "F.Cu" "B.Cu") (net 8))
 (via (at 35.306 7.62) (size 0.6) (drill 0.3) (layers "F.Cu" "B.Cu") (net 7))
 (via (at 31.242 26.67) (size 0.6) (drill 0.3) (layers "F.Cu" "B.Cu") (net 4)) (gr_line (start 0 0) (end 47 0) (layer "Edge.Cuts"))
 (gr_line (start 47 0) (end 47 33) (layer "Edge.Cuts")) (gr_line (start 47 33) (end 0 33) (layer "Edge.Cuts"))
 (gr_line (start 0 33) (end 0 0) (layer "Edge.Cuts")))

